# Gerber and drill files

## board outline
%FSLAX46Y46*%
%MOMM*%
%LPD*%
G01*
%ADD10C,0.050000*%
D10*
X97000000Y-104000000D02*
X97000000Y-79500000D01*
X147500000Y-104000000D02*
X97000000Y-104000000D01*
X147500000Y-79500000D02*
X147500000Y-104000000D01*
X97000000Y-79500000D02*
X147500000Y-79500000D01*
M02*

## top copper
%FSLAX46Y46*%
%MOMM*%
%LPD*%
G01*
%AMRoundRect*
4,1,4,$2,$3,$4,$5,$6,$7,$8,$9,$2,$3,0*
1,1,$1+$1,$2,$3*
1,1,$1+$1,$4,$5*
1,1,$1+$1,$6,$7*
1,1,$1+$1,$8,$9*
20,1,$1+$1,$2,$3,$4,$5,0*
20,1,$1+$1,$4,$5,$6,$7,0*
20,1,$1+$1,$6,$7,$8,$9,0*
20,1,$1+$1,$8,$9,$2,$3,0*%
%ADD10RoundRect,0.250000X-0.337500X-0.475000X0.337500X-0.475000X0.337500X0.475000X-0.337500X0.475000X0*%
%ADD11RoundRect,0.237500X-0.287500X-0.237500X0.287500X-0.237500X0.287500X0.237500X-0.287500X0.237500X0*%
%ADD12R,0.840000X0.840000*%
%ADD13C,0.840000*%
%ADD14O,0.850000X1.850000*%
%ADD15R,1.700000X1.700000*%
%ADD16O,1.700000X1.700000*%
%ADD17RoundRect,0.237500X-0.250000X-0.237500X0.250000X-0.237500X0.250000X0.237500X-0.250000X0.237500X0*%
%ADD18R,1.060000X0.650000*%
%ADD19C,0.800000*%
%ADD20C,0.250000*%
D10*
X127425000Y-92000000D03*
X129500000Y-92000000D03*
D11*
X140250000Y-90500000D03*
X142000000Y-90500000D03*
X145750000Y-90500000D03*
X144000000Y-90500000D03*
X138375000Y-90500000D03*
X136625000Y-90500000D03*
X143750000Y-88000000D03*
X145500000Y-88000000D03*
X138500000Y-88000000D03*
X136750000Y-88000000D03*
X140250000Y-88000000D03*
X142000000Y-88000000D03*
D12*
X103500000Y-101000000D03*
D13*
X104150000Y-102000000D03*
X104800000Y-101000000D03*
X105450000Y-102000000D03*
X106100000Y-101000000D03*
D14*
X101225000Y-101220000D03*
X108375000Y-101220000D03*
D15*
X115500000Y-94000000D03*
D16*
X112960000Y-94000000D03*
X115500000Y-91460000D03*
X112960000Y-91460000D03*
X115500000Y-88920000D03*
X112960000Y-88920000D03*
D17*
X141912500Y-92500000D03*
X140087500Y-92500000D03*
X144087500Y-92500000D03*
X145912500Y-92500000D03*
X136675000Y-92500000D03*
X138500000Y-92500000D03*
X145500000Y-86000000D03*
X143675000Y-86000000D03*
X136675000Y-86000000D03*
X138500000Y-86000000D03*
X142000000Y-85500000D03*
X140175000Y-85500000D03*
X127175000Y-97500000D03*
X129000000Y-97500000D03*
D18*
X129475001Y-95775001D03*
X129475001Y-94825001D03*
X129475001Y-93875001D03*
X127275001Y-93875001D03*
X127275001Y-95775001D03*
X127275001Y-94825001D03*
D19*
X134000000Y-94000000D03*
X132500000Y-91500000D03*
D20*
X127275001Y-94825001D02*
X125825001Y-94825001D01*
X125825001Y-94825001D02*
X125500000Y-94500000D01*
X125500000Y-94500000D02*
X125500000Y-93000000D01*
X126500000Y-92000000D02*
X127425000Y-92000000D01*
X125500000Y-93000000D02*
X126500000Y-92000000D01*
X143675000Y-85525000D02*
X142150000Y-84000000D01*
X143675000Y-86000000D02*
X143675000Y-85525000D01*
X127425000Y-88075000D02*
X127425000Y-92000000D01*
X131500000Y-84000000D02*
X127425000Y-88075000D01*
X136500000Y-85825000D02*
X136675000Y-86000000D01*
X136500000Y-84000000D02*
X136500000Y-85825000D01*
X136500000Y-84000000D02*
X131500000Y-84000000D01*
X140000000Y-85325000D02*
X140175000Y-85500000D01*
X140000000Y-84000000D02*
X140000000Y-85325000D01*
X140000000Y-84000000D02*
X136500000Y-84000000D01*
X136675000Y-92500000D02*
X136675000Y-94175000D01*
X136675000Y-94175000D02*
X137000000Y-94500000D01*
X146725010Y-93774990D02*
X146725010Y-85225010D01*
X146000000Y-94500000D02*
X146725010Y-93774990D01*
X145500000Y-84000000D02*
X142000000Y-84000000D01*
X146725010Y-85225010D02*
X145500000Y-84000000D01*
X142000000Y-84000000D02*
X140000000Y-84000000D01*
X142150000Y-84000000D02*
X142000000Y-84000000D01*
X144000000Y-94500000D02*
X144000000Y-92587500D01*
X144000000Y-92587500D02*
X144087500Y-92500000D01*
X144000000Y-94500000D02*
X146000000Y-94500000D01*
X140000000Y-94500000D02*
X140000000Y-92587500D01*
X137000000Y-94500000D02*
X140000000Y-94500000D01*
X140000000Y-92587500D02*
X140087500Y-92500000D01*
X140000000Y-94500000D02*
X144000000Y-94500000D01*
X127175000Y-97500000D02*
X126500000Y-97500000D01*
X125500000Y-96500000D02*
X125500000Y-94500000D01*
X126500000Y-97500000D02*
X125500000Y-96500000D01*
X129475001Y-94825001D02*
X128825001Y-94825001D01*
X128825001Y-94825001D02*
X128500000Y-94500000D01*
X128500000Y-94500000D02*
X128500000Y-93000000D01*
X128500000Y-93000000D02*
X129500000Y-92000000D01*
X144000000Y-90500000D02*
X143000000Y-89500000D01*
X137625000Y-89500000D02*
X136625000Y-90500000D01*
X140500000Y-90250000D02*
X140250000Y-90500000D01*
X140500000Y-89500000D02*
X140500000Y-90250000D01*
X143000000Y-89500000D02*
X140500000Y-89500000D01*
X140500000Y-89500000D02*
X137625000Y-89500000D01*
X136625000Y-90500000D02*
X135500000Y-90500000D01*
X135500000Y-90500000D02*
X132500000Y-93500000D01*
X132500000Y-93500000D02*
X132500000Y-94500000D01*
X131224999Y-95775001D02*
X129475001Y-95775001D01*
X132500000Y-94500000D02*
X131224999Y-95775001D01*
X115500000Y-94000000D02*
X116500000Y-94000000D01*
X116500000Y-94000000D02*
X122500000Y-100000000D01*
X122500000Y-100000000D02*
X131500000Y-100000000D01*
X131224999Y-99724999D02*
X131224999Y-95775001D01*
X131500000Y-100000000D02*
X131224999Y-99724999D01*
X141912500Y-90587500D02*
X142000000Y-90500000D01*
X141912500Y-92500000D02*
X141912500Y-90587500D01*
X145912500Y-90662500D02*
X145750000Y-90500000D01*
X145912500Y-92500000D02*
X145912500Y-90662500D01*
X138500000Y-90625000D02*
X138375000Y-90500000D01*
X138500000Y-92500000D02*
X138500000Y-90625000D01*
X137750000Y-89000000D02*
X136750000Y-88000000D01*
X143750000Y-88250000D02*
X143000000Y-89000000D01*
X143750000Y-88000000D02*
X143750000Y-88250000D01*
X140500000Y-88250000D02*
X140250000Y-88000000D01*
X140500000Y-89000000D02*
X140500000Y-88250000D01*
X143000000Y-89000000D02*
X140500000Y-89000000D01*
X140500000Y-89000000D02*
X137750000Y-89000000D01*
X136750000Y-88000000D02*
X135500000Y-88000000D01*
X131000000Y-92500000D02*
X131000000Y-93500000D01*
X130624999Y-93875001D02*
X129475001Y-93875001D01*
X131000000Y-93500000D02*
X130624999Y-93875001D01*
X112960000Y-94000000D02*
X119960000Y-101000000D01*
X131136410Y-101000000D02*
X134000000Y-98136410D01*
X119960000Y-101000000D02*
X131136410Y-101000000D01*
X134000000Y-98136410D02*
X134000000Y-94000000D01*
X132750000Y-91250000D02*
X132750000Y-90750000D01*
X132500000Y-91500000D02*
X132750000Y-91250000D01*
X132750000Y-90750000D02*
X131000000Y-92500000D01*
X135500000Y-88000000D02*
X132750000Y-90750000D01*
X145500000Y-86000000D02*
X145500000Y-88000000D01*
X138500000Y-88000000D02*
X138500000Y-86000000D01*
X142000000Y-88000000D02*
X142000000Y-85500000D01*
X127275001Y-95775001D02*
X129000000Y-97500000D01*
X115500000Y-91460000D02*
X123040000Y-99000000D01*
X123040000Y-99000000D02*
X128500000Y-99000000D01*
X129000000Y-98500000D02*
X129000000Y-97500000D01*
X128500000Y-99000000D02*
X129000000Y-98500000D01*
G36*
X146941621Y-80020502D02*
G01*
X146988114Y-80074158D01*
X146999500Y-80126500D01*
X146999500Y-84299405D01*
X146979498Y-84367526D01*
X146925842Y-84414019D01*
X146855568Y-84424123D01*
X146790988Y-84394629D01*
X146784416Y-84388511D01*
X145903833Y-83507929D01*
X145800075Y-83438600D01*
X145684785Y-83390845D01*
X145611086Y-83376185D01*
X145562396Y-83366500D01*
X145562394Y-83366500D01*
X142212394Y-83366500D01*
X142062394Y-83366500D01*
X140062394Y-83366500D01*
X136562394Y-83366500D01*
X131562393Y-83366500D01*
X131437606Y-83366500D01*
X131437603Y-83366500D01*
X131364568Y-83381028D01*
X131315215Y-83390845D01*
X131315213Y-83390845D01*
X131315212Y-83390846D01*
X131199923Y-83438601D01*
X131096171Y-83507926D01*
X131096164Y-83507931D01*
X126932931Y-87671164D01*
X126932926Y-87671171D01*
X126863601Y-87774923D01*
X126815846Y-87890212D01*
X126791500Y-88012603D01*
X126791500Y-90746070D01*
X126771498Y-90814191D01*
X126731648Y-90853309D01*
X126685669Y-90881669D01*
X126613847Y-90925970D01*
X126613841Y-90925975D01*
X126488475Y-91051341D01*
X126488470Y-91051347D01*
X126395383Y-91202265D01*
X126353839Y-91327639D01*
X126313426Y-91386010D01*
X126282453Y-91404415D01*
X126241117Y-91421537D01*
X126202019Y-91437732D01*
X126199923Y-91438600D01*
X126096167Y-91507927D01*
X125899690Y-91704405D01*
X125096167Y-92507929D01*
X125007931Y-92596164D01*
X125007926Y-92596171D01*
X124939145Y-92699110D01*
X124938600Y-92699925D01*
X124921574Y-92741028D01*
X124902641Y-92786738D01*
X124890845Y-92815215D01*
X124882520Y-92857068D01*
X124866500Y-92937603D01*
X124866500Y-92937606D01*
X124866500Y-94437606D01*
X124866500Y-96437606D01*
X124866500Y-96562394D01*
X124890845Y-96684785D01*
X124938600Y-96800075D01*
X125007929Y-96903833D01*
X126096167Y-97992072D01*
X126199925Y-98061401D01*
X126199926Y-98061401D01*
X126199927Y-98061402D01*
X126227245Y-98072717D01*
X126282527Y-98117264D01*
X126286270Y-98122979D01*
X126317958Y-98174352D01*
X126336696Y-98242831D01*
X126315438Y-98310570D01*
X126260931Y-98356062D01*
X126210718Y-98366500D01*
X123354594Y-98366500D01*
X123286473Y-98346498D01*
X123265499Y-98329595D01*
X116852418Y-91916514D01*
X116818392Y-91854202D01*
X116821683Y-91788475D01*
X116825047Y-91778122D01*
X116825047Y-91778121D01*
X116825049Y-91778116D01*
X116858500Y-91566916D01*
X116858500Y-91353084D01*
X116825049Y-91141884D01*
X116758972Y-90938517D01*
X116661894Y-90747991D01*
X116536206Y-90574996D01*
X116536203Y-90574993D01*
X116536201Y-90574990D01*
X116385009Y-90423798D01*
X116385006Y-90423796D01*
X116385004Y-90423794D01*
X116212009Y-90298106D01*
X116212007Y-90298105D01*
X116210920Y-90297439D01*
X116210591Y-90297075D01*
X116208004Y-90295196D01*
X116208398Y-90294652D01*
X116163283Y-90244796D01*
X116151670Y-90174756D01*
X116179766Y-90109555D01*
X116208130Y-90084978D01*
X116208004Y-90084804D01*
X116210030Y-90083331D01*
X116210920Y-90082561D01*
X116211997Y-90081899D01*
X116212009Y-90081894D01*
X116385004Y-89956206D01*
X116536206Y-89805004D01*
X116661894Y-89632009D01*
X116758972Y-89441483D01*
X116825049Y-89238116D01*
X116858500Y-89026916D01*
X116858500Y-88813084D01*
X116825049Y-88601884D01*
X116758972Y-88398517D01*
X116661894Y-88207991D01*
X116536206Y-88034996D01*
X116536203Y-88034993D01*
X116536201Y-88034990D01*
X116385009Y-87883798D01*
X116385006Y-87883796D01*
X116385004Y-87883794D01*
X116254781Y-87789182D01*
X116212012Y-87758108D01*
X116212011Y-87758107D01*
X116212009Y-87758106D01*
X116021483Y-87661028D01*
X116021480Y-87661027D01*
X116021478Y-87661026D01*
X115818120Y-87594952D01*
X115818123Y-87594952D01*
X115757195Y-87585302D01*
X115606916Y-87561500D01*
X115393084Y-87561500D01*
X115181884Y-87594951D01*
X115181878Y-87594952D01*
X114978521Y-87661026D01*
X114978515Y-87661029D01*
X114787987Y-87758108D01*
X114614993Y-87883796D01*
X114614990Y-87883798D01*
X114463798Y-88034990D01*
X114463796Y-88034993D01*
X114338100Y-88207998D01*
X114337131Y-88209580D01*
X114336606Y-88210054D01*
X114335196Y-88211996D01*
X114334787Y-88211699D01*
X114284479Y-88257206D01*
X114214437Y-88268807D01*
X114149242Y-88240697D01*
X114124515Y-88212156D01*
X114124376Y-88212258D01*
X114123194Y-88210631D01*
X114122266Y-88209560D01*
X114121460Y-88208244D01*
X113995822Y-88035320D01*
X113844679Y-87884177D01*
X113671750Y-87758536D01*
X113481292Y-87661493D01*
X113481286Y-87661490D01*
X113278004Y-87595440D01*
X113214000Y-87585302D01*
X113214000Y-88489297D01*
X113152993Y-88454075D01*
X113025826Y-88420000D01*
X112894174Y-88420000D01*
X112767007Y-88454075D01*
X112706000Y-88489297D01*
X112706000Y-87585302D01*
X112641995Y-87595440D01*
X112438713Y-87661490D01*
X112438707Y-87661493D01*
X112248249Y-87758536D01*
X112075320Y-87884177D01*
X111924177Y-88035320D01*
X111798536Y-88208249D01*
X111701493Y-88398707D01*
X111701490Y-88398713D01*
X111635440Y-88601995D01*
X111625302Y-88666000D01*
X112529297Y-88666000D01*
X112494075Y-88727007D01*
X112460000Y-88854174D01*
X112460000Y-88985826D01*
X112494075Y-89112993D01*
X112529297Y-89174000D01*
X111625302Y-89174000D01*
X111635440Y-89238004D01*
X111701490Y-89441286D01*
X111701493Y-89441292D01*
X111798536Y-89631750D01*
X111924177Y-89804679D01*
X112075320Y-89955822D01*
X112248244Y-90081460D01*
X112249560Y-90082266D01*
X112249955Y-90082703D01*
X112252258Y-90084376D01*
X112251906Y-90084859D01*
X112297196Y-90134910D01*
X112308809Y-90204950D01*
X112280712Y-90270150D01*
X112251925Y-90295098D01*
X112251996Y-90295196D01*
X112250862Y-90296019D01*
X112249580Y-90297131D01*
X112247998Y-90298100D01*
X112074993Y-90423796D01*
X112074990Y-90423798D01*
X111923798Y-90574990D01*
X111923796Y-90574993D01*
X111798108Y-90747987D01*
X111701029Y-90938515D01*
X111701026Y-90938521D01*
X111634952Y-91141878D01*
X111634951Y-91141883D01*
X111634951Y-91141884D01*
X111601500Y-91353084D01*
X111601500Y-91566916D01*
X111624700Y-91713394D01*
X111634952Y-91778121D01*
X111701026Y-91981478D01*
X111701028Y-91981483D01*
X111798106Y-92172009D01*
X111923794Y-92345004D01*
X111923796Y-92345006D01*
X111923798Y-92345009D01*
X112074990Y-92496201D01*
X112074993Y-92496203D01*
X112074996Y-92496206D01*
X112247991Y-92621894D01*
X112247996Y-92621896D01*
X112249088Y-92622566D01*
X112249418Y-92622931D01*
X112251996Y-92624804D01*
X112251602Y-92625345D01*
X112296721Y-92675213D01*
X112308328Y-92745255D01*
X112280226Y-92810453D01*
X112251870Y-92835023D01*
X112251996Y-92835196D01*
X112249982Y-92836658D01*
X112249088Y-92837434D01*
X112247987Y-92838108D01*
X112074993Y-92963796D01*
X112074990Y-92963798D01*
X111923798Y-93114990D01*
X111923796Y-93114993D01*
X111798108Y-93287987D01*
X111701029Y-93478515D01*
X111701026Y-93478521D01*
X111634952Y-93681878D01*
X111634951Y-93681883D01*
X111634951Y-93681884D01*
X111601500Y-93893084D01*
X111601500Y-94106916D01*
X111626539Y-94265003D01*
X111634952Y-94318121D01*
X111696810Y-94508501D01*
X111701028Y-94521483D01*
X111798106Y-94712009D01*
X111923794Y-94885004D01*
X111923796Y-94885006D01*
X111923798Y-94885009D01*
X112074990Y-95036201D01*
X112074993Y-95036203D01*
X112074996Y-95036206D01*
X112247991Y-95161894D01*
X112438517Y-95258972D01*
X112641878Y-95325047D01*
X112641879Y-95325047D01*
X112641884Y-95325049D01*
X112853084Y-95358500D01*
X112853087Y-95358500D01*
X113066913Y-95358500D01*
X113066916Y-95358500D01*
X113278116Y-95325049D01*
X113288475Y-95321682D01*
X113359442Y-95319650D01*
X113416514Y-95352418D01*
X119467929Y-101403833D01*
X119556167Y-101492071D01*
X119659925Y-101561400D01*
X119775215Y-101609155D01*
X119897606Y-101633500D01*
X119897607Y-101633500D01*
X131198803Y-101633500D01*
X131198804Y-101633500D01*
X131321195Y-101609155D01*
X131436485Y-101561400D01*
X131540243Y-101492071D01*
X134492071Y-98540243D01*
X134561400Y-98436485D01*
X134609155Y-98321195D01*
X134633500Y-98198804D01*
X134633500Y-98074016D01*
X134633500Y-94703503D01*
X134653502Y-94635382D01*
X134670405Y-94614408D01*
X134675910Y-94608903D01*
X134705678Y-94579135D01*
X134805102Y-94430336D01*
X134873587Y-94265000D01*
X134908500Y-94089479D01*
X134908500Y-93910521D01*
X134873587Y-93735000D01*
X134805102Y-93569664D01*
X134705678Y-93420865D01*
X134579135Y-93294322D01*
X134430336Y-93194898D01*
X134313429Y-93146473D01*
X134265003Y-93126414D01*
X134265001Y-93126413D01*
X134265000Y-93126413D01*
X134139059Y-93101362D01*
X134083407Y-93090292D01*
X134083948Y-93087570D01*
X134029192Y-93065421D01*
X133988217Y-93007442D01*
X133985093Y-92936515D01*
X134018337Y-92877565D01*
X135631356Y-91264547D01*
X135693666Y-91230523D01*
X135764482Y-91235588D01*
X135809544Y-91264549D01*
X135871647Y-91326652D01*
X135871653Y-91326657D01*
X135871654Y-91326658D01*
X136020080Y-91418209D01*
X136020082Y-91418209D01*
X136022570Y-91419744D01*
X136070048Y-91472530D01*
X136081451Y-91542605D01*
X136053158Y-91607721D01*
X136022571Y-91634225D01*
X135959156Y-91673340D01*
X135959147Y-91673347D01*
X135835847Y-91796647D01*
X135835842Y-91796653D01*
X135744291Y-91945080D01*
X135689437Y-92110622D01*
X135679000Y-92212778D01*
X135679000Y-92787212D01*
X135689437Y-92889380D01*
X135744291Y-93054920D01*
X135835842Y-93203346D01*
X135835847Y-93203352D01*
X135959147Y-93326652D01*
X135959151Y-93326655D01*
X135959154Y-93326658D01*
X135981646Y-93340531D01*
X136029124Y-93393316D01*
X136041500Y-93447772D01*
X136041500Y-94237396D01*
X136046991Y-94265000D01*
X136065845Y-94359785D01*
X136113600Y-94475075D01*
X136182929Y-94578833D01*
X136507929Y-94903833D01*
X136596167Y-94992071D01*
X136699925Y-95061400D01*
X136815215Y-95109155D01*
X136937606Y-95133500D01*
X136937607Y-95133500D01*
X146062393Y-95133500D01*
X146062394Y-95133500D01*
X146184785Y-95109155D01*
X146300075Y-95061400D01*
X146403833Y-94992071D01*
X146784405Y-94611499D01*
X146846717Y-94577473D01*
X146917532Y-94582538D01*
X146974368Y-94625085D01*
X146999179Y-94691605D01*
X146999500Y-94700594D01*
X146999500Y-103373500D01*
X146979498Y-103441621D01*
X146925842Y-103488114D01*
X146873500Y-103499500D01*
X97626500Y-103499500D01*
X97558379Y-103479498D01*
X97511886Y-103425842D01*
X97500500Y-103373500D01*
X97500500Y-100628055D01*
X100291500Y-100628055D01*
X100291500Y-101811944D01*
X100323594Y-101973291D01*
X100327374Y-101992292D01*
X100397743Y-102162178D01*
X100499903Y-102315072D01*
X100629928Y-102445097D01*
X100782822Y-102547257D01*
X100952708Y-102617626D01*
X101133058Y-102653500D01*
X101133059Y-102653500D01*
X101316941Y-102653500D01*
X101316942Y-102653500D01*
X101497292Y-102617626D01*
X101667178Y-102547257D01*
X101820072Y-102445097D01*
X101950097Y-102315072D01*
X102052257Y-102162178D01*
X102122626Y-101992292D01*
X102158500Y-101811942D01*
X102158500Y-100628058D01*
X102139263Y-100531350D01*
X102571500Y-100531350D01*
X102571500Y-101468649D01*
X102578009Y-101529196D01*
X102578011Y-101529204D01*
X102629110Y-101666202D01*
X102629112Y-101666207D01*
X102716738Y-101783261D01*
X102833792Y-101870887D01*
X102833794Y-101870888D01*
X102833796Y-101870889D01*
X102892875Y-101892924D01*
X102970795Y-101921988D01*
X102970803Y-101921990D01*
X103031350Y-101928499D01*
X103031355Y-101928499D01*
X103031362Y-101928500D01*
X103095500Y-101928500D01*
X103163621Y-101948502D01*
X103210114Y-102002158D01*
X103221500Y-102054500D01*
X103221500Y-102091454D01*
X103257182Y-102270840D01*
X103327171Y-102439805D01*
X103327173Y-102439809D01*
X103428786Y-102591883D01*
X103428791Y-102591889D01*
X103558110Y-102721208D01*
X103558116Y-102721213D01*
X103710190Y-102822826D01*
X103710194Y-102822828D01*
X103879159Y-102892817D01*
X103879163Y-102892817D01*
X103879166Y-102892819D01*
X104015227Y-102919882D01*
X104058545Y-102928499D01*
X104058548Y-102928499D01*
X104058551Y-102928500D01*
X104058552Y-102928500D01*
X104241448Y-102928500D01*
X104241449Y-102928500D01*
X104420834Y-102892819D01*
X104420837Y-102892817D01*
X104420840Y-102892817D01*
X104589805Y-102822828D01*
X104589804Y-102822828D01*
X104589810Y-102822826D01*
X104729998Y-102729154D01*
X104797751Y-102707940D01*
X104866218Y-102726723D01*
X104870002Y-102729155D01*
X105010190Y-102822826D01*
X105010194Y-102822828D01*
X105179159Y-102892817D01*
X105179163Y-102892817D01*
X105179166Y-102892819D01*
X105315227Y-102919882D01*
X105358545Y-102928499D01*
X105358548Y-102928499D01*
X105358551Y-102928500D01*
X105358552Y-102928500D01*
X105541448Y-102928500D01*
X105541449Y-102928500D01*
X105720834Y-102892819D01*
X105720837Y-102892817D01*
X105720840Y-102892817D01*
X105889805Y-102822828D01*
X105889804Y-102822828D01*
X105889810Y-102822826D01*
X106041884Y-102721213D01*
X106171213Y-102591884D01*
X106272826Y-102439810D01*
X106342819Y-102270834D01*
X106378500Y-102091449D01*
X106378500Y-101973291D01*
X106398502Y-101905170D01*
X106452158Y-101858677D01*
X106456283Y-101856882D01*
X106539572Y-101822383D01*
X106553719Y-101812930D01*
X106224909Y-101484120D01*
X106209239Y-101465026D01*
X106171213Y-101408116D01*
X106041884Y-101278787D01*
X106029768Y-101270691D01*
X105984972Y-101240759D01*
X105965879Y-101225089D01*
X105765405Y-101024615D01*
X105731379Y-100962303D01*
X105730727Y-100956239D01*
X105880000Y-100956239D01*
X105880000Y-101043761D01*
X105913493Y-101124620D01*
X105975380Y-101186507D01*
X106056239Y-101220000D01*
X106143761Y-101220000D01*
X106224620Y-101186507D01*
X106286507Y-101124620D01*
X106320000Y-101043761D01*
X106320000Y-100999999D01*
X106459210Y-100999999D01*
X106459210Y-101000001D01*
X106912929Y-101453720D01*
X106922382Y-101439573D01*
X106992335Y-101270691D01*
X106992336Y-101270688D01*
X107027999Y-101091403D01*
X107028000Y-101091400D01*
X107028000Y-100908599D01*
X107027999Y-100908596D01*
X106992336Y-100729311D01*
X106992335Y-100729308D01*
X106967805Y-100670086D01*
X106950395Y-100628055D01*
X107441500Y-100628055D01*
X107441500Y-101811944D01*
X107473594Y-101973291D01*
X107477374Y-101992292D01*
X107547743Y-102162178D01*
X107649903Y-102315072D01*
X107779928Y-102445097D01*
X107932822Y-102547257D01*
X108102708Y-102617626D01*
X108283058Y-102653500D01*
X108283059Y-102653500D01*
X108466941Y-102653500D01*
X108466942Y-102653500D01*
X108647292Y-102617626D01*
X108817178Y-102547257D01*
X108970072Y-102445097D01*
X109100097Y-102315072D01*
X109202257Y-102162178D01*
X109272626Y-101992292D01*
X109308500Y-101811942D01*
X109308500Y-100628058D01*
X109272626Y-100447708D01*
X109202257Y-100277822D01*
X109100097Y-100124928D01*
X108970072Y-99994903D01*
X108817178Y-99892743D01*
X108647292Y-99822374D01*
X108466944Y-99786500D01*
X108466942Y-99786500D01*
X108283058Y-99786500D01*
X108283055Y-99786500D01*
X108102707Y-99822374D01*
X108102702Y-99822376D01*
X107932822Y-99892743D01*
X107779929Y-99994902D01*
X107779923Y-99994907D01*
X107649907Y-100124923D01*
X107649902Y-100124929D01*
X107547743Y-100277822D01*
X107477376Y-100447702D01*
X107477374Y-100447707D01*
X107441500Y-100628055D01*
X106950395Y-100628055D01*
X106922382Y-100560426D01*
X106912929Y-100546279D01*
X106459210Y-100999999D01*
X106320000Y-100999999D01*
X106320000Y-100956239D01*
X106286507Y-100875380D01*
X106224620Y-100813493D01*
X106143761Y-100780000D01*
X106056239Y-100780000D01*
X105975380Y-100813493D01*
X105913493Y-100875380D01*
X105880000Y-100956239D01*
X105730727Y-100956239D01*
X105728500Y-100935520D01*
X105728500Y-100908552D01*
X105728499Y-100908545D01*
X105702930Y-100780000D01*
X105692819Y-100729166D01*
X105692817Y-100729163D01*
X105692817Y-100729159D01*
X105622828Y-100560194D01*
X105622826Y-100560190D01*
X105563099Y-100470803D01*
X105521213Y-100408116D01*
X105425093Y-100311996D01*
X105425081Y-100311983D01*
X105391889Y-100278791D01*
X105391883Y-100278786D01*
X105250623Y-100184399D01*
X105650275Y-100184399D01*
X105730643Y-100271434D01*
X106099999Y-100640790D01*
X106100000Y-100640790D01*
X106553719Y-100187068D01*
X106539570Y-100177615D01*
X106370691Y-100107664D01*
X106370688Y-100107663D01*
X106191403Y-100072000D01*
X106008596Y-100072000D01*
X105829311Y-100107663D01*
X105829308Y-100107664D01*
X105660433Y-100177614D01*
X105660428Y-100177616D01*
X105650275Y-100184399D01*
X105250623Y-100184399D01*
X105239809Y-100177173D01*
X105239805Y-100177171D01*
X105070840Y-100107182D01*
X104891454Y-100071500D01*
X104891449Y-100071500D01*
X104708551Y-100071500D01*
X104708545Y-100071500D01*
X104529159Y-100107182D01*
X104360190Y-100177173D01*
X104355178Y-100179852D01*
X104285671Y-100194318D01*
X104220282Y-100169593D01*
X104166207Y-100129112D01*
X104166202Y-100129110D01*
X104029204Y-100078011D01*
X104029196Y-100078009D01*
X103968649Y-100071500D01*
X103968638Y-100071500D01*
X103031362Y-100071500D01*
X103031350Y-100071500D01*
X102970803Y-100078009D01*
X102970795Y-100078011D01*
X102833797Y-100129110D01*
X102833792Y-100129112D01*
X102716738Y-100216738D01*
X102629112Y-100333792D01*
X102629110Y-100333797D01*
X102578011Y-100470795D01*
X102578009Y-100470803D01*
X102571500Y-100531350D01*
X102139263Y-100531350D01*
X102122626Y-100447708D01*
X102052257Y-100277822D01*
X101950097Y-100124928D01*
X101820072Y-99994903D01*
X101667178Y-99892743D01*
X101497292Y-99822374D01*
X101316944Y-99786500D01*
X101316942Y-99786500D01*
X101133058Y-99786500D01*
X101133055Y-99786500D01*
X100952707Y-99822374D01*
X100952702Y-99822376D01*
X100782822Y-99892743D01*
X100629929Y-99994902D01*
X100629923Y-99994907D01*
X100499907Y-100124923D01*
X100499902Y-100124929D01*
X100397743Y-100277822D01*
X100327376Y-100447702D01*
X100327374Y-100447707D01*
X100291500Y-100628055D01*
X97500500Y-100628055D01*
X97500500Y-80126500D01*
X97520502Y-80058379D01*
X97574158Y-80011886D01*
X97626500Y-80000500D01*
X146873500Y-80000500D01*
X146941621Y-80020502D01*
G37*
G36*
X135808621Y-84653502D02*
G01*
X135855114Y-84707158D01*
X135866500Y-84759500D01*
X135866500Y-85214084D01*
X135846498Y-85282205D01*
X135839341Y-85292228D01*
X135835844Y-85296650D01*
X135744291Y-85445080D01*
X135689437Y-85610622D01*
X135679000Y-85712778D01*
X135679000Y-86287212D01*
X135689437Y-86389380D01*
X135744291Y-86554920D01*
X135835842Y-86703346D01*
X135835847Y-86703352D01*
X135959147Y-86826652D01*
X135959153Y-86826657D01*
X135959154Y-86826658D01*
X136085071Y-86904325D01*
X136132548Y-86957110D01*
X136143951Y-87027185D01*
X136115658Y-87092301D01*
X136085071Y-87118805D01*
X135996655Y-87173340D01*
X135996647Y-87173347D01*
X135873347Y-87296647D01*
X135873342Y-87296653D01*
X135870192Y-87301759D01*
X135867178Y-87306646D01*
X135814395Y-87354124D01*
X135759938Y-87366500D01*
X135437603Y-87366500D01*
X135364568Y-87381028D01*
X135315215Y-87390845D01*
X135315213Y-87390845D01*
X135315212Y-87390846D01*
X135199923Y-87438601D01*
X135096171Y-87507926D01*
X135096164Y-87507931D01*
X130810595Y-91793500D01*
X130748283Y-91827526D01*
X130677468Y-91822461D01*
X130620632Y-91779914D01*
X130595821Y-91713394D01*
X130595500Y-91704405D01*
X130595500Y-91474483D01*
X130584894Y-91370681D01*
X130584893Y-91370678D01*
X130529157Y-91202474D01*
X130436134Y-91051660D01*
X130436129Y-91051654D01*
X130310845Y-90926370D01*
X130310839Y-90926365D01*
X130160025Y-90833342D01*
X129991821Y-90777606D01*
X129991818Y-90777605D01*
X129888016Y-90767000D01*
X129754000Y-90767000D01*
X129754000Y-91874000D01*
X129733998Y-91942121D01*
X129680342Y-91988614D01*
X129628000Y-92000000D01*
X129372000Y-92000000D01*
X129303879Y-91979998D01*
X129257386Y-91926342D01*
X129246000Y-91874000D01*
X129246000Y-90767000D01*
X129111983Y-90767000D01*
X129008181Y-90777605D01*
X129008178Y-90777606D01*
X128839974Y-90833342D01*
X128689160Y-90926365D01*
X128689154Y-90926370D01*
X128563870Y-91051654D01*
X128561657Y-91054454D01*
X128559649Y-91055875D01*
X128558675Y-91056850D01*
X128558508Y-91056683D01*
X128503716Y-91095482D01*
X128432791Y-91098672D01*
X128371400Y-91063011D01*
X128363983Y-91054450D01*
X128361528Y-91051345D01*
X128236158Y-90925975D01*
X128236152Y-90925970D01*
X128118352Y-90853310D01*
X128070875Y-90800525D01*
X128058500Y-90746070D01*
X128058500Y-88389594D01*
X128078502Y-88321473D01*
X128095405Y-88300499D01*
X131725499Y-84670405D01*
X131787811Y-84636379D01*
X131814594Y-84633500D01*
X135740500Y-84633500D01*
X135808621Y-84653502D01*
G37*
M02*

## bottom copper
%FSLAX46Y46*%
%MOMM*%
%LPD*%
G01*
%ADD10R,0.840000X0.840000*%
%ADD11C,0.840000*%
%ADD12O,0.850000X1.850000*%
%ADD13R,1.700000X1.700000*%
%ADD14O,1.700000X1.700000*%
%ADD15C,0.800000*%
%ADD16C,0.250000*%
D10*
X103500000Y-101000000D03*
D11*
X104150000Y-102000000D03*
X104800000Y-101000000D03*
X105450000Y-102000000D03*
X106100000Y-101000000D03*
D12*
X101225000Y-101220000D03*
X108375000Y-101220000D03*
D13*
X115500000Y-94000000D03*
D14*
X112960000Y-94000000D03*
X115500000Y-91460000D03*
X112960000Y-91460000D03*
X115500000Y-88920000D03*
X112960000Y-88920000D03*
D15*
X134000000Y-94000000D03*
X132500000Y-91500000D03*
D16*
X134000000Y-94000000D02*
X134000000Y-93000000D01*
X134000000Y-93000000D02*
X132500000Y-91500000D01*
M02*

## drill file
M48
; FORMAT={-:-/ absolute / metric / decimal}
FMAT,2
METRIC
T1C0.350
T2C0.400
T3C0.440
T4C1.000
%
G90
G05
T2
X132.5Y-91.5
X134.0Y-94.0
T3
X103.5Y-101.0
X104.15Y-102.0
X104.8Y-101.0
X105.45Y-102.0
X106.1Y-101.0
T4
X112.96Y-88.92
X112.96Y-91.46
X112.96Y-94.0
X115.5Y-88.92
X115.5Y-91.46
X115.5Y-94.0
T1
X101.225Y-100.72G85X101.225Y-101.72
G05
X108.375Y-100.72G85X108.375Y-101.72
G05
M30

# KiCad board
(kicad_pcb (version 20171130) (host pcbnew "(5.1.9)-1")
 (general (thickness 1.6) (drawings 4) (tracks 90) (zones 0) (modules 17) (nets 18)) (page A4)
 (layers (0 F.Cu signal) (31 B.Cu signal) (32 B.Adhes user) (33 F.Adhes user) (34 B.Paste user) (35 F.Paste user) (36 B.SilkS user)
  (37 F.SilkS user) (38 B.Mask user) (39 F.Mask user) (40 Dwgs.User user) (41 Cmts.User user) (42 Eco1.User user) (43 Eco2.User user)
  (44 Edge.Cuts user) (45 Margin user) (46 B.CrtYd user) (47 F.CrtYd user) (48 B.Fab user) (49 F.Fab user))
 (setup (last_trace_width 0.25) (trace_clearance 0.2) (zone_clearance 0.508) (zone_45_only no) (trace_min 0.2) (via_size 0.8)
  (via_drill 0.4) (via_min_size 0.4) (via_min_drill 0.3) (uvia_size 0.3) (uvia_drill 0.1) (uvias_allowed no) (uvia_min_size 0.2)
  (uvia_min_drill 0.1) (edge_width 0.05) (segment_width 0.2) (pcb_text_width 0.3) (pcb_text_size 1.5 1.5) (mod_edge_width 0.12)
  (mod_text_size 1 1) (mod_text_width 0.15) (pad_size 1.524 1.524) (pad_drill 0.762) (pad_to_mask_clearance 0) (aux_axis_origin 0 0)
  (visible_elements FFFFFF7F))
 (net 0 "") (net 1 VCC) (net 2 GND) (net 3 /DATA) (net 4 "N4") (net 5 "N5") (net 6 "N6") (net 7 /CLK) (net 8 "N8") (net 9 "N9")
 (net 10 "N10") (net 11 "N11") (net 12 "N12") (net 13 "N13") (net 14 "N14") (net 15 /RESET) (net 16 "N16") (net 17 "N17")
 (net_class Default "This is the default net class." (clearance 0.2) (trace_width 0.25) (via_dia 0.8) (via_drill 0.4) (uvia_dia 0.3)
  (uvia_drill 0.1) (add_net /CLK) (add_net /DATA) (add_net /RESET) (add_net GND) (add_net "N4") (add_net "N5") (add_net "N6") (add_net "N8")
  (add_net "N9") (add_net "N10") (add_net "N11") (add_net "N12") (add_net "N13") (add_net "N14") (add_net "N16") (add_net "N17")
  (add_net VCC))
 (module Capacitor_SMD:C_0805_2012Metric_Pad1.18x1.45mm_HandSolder (layer F.Cu) (at 128.4625 92)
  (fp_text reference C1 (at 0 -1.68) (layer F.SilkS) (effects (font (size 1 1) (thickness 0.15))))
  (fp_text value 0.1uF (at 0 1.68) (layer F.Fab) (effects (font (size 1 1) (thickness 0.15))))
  (pad 1 smd roundrect (at -1.0375 0) (size 1.175 1.45) (layers F.Cu F.Paste F.Mask) (roundrect_rratio 0.212766) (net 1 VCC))
  (pad 2 smd roundrect (at 1.0375 0) (size 1.175 1.45) (layers F.Cu F.Paste F.Mask) (roundrect_rratio 0.212766) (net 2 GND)))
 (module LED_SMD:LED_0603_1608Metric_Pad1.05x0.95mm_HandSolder (layer F.Cu) (at 141.125 90.5)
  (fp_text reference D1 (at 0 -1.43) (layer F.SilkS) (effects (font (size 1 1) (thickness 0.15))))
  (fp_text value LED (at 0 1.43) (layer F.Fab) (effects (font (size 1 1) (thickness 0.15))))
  (pad 1 smd roundrect (at -0.875 0) (size 1.05 0.95) (layers F.Cu F.Paste F.Mask) (roundrect_rratio 0.25) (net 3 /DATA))
  (pad 2 smd roundrect (at 0.875 0) (size 1.05 0.95) (layers F.Cu F.Paste F.Mask) (roundrect_rratio 0.25) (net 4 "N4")))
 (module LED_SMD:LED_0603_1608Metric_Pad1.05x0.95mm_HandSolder (layer F.Cu) (at 144.875 90.5)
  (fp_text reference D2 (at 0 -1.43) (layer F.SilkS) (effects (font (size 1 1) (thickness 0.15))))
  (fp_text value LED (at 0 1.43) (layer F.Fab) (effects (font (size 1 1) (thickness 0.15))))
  (pad 2 smd roundrect (at 0.875 0) (size 1.05 0.95) (layers F.Cu F.Paste F.Mask) (roundrect_rratio 0.25) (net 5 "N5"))
  (pad 1 smd roundrect (at -0.875 0) (size 1.05 0.95) (layers F.Cu F.Paste F.Mask) (roundrect_rratio 0.25) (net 3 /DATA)))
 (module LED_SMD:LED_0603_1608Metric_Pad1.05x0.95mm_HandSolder (layer F.Cu) (at 137.5 90.5)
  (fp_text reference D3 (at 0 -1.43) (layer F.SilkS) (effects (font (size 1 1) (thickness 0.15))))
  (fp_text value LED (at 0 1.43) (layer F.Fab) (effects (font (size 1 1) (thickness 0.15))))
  (pad 2 smd roundrect (at 0.875 0) (size 1.05 0.95) (layers F.Cu F.Paste F.Mask) (roundrect_rratio 0.25) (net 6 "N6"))
  (pad 1 smd roundrect (at -0.875 0) (size 1.05 0.95) (layers F.Cu F.Paste F.Mask) (roundrect_rratio 0.25) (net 3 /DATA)))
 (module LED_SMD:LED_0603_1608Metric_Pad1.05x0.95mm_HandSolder (layer F.Cu) (at 144.625 88)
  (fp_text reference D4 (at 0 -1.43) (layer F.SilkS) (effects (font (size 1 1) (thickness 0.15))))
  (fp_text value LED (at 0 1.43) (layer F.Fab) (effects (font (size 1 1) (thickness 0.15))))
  (pad 1 smd roundrect (at -0.875 0) (size 1.05 0.95) (layers F.Cu F.Paste F.Mask) (roundrect_rratio 0.25) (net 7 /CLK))
  (pad 2 smd roundrect (at 0.875 0) (size 1.05 0.95) (layers F.Cu F.Paste F.Mask) (roundrect_rratio 0.25) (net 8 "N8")))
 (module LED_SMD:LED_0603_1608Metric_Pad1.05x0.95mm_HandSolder (layer F.Cu) (at 137.625 88)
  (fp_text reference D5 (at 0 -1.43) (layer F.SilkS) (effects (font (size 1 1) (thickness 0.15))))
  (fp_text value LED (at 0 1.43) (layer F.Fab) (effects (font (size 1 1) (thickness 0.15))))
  (pad 2 smd roundrect (at 0.875 0) (size 1.05 0.95) (layers F.Cu F.Paste F.Mask) (roundrect_rratio 0.25) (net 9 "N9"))
  (pad 1 smd roundrect (at -0.875 0) (size 1.05 0.95) (layers F.Cu F.Paste F.Mask) (roundrect_rratio 0.25) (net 7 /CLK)))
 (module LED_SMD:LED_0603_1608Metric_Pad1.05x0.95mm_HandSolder (layer F.Cu) (at 141.125 88)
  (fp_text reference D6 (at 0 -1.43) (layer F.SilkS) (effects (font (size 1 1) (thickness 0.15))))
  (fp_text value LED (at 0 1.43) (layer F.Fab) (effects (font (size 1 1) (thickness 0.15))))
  (pad 1 smd roundrect (at -0.875 0) (size 1.05 0.95) (layers F.Cu F.Paste F.Mask) (roundrect_rratio 0.25) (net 7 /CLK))
  (pad 2 smd roundrect (at 0.875 0) (size 1.05 0.95) (layers F.Cu F.Paste F.Mask) (roundrect_rratio 0.25) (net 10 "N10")))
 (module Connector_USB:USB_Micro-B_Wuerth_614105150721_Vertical (layer F.Cu) (at 103.5 101)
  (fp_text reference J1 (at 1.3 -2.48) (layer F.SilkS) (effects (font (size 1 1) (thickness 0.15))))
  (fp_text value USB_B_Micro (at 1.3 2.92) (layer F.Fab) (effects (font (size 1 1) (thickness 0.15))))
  (pad 1 thru_hole rect (at 0 0) (size 0.84 0.84) (drill 0.44) (layers *.Cu *.Mask) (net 1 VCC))
  (pad 2 thru_hole circle (at 0.65 1) (size 0.84 0.84) (drill 0.44) (layers *.Cu *.Mask) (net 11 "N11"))
  (pad 3 thru_hole circle (at 1.3 0) (size 0.84 0.84) (drill 0.44) (layers *.Cu *.Mask) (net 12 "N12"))
  (pad 4 thru_hole circle (at 1.95 1) (size 0.84 0.84) (drill 0.44) (layers *.Cu *.Mask) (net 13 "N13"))
  (pad 5 thru_hole circle (at 2.6 0) (size 0.84 0.84) (drill 0.44) (layers *.Cu *.Mask) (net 2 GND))
  (pad 6 thru_hole oval (at -2.275 0.22) (size 0.85 1.85) (drill oval 0.35 1.35) (layers *.Cu *.Mask) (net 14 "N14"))
  (pad 6 thru_hole oval (at 4.875 0.22) (size 0.85 1.85) (drill oval 0.35 1.35) (layers *.Cu *.Mask) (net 14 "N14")))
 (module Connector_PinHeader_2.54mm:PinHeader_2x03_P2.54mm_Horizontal (layer F.Cu) (at 115.5 94 180)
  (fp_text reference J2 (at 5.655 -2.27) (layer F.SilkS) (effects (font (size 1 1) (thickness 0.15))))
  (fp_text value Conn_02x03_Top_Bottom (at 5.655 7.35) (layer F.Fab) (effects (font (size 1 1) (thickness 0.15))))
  (pad 1 thru_hole rect (at 0 0 180) (size 1.7 1.7) (drill 1) (layers *.Cu *.Mask) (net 3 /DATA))
  (pad 2 thru_hole oval (at 2.54 0 180) (size 1.7 1.7) (drill 1) (layers *.Cu *.Mask) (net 7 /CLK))
  (pad 3 thru_hole oval (at 0 2.54 180) (size 1.7 1.7) (drill 1) (layers *.Cu *.Mask) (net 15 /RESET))
  (pad 4 thru_hole oval (at 2.54 2.54 180) (size 1.7 1.7) (drill 1) (layers *.Cu *.Mask) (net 1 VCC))
  (pad 5 thru_hole oval (at 0 5.08 180) (size 1.7 1.7) (drill 1) (layers *.Cu *.Mask) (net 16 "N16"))
  (pad 6 thru_hole oval (at 2.54 5.08 180) (size 1.7 1.7) (drill 1) (layers *.Cu *.Mask) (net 2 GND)))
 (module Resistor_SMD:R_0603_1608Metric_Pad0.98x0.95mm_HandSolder (layer F.Cu) (at 141 92.5)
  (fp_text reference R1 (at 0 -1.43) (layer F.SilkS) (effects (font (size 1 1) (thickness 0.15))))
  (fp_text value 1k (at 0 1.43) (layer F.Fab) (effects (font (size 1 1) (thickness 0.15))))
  (pad 2 smd roundrect (at 0.9125 0) (size 0.975 0.95) (layers F.Cu F.Paste F.Mask) (roundrect_rratio 0.25) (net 4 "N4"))
  (pad 1 smd roundrect (at -0.9125 0) (size 0.975 0.95) (layers F.Cu F.Paste F.Mask) (roundrect_rratio 0.25) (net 1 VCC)))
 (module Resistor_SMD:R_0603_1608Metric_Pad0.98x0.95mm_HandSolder (layer F.Cu) (at 145 92.5)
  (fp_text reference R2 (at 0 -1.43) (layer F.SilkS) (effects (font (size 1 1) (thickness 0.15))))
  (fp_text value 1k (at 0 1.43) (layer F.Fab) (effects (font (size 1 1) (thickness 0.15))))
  (pad 1 smd roundrect (at -0.9125 0) (size 0.975 0.95) (layers F.Cu F.Paste F.Mask) (roundrect_rratio 0.25) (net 1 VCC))
  (pad 2 smd roundrect (at 0.9125 0) (size 0.975 0.95) (layers F.Cu F.Paste F.Mask) (roundrect_rratio 0.25) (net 5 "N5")))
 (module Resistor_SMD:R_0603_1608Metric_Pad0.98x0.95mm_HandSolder (layer F.Cu) (at 137.5875 92.5)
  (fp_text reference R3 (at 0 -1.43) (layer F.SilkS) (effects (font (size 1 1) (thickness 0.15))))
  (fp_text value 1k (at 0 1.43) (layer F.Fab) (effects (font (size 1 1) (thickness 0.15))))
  (pad 1 smd roundrect (at -0.9125 0) (size 0.975 0.95) (layers F.Cu F.Paste F.Mask) (roundrect_rratio 0.25) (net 1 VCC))
  (pad 2 smd roundrect (at 0.9125 0) (size 0.975 0.95) (layers F.Cu F.Paste F.Mask) (roundrect_rratio 0.25) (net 6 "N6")))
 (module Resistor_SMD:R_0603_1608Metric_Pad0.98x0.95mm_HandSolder (layer F.Cu) (at 144.5875 86)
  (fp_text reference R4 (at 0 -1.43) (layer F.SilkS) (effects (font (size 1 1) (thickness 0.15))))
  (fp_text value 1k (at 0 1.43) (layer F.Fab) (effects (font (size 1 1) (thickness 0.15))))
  (pad 2 smd roundrect (at 0.9125 0) (size 0.975 0.95) (layers F.Cu F.Paste F.Mask) (roundrect_rratio 0.25) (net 8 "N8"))
  (pad 1 smd roundrect (at -0.9125 0) (size 0.975 0.95) (layers F.Cu F.Paste F.Mask) (roundrect_rratio 0.25) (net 1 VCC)))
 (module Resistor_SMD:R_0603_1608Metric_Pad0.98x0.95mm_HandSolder (layer F.Cu) (at 137.5875 86)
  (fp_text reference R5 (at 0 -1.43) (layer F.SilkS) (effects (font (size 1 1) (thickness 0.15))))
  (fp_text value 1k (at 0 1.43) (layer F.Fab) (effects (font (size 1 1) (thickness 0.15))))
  (pad 1 smd roundrect (at -0.9125 0) (size 0.975 0.95) (layers F.Cu F.Paste F.Mask) (roundrect_rratio 0.25) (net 1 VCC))
  (pad 2 smd roundrect (at 0.9125 0) (size 0.975 0.95) (layers F.Cu F.Paste F.Mask) (roundrect_rratio 0.25) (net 9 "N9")))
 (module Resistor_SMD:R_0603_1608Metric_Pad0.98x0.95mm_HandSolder (layer F.Cu) (at 141.0875 85.5)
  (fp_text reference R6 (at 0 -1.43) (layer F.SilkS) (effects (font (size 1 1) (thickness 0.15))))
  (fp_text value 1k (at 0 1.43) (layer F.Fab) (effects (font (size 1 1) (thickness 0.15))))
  (pad 2 smd roundrect (at 0.9125 0) (size 0.975 0.95) (layers F.Cu F.Paste F.Mask) (roundrect_rratio 0.25) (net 10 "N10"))
  (pad 1 smd roundrect (at -0.9125 0) (size 0.975 0.95) (layers F.Cu F.Paste F.Mask) (roundrect_rratio 0.25) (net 1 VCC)))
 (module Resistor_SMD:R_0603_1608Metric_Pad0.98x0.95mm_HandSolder (layer F.Cu) (at 128.0875 97.5)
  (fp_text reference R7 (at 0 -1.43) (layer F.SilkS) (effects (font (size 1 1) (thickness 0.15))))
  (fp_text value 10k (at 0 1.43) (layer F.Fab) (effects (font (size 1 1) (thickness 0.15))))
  (pad 1 smd roundrect (at -0.9125 0) (size 0.975 0.95) (layers F.Cu F.Paste F.Mask) (roundrect_rratio 0.25) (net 1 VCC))
  (pad 2 smd roundrect (at 0.9125 0) (size 0.975 0.95) (layers F.Cu F.Paste F.Mask) (roundrect_rratio 0.25) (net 15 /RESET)))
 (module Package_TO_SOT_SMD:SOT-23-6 (layer F.Cu) (at 128.375001 94.825001 180)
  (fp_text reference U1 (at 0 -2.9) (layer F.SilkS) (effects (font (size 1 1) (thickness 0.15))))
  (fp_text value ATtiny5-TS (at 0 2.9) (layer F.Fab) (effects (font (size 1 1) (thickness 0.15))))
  (pad 1 smd rect (at -1.1 -0.95 180) (size 1.06 0.65) (layers F.Cu F.Paste F.Mask) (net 3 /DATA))
  (pad 2 smd rect (at -1.1 0 180) (size 1.06 0.65) (layers F.Cu F.Paste F.Mask) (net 2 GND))
  (pad 3 smd rect (at -1.1 0.95 180) (size 1.06 0.65) (layers F.Cu F.Paste F.Mask) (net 7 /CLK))
  (pad 4 smd rect (at 1.1 0.95 180) (size 1.06 0.65) (layers F.Cu F.Paste F.Mask) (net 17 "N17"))
  (pad 6 smd rect (at 1.1 -0.95 180) (size 1.06 0.65) (layers F.Cu F.Paste F.Mask) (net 15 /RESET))
  (pad 5 smd rect (at 1.1 0 180) (size 1.06 0.65) (layers F.Cu F.Paste F.Mask) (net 1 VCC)))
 (gr_line (start 97 104) (end 97 79.5) (layer Edge.Cuts) (width 0.05))
 (gr_line (start 147.5 104) (end 97 104) (layer Edge.Cuts) (width 0.05))
 (gr_line (start 147.5 79.5) (end 147.5 104) (layer Edge.Cuts) (width 0.05))
 (gr_line (start 97 79.5) (end 147.5 79.5) (layer Edge.Cuts) (width 0.05))
 (segment (start 127.275001 94.825001) (end 125.825001 94.825001) (width 0.25) (layer F.Cu) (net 1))
 (segment (start 125.825001 94.825001) (end 125.5 94.5) (width 0.25) (layer F.Cu) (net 1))
 (segment (start 125.5 94.5) (end 125.5 93) (width 0.25) (layer F.Cu) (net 1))
 (segment (start 126.5 92) (end 127.425 92) (width 0.25) (layer F.Cu) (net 1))
 (segment (start 125.5 93) (end 126.5 92) (width 0.25) (layer F.Cu) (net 1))
 (segment (start 143.675 85.525) (end 142.15 84) (width 0.25) (layer F.Cu) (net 1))
 (segment (start 143.675 86) (end 143.675 85.525) (width 0.25) (layer F.Cu) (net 1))
 (segment (start 127.425 88.075) (end 127.425 92) (width 0.25) (layer F.Cu) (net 1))
 (segment (start 131.5 84) (end 127.425 88.075) (width 0.25) (layer F.Cu) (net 1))
 (segment (start 136.5 85.825) (end 136.675 86) (width 0.25) (layer F.Cu) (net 1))
 (segment (start 136.5 84) (end 136.5 85.825) (width 0.25) (layer F.Cu) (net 1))
 (segment (start 136.5 84) (end 131.5 84) (width 0.25) (layer F.Cu) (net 1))
 (segment (start 140 85.325) (end 140.175 85.5) (width 0.25) (layer F.Cu) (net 1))
 (segment (start 140 84) (end 140 85.325) (width 0.25) (layer F.Cu) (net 1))
 (segment (start 140 84) (end 136.5 84) (width 0.25) (layer F.Cu) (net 1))
 (segment (start 136.675 92.5) (end 136.675 94.175) (width 0.25) (layer F.Cu) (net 1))
 (segment (start 136.675 94.175) (end 137 94.5) (width 0.25) (layer F.Cu) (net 1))
 (segment (start 146.72501 93.77499) (end 146.72501 85.22501) (width 0.25) (layer F.Cu) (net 1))
 (segment (start 146 94.5) (end 146.72501 93.77499) (width 0.25) (layer F.Cu) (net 1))
 (segment (start 145.5 84) (end 142 84) (width 0.25) (layer F.Cu) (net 1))
 (segment (start 146.72501 85.22501) (end 145.5 84) (width 0.25) (layer F.Cu) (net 1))
 (segment (start 142 84) (end 140 84) (width 0.25) (layer F.Cu) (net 1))
 (segment (start 142.15 84) (end 142 84) (width 0.25) (layer F.Cu) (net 1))
 (segment (start 144 94.5) (end 144 92.5875) (width 0.25) (layer F.Cu) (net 1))
 (segment (start 144 92.5875) (end 144.0875 92.5) (width 0.25) (layer F.Cu) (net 1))
 (segment (start 144 94.5) (end 146 94.5) (width 0.25) (layer F.Cu) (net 1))
 (segment (start 140 94.5) (end 140 92.5875) (width 0.25) (layer F.Cu) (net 1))
 (segment (start 137 94.5) (end 140 94.5) (width 0.25) (layer F.Cu) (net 1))
 (segment (start 140 92.5875) (end 140.0875 92.5) (width 0.25) (layer F.Cu) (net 1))
 (segment (start 140 94.5) (end 144 94.5) (width 0.25) (layer F.Cu) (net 1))
 (segment (start 127.175 97.5) (end 126.5 97.5) (width 0.25) (layer F.Cu) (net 1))
 (segment (start 125.5 96.5) (end 125.5 94.5) (width 0.25) (layer F.Cu) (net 1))
 (segment (start 126.5 97.5) (end 125.5 96.5) (width 0.25) (layer F.Cu) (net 1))
 (segment (start 129.475001 94.825001) (end 128.825001 94.825001) (width 0.25) (layer F.Cu) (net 2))
 (segment (start 128.825001 94.825001) (end 128.5 94.5) (width 0.25) (layer F.Cu) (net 2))
 (segment (start 128.5 94.5) (end 128.5 93) (width 0.25) (layer F.Cu) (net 2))
 (segment (start 128.5 93) (end 129.5 92) (width 0.25) (layer F.Cu) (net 2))
 (segment (start 144 90.5) (end 143 89.5) (width 0.25) (layer F.Cu) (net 3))
 (segment (start 137.625 89.5) (end 136.625 90.5) (width 0.25) (layer F.Cu) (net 3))
 (segment (start 140.5 90.25) (end 140.25 90.5) (width 0.25) (layer F.Cu) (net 3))
 (segment (start 140.5 89.5) (end 140.5 90.25) (width 0.25) (layer F.Cu) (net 3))
 (segment (start 143 89.5) (end 140.5 89.5) (width 0.25) (layer F.Cu) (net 3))
 (segment (start 140.5 89.5) (end 137.625 89.5) (width 0.25) (layer F.Cu) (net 3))
 (segment (start 136.625 90.5) (end 135.5 90.5) (width 0.25) (layer F.Cu) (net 3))
 (segment (start 135.5 90.5) (end 132.5 93.5) (width 0.25) (layer F.Cu) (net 3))
 (segment (start 132.5 93.5) (end 132.5 94.5) (width 0.25) (layer F.Cu) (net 3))
 (segment (start 131.224999 95.775001) (end 129.475001 95.775001) (width 0.25) (layer F.Cu) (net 3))
 (segment (start 132.5 94.5) (end 131.224999 95.775001) (width 0.25) (layer F.Cu) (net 3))
 (segment (start 115.5 94) (end 116.5 94) (width 0.25) (layer F.Cu) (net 3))
 (segment (start 116.5 94) (end 122.5 100) (width 0.25) (layer F.Cu) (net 3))
 (segment (start 122.5 100) (end 131.5 100) (width 0.25) (layer F.Cu) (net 3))
 (segment (start 131.224999 99.724999) (end 131.224999 95.775001) (width 0.25) (layer F.Cu) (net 3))
 (segment (start 131.5 100) (end 131.224999 99.724999) (width 0.25) (layer F.Cu) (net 3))
 (segment (start 141.9125 90.5875) (end 142 90.5) (width 0.25) (layer F.Cu) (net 4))
 (segment (start 141.9125 92.5) (end 141.9125 90.5875) (width 0.25) (layer F.Cu) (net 4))
 (segment (start 145.9125 90.6625) (end 145.75 90.5) (width 0.25) (layer F.Cu) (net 5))
 (segment (start 145.9125 92.5) (end 145.9125 90.6625) (width 0.25) (layer F.Cu) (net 5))
 (segment (start 138.5 90.625) (end 138.375 90.5) (width 0.25) (layer F.Cu) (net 6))
 (segment (start 138.5 92.5) (end 138.5 90.625) (width 0.25) (layer F.Cu) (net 6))
 (segment (start 137.75 89) (end 136.75 88) (width 0.25) (layer F.Cu) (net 7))
 (segment (start 143.75 88.25) (end 143 89) (width 0.25) (layer F.Cu) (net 7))
 (segment (start 143.75 88) (end 143.75 88.25) (width 0.25) (layer F.Cu) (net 7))
 (segment (start 140.5 88.25) (end 140.25 88) (width 0.25) (layer F.Cu) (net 7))
 (segment (start 140.5 89) (end 140.5 88.25) (width 0.25) (layer F.Cu) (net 7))
 (segment (start 143 89) (end 140.5 89) (width 0.25) (layer F.Cu) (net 7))
 (segment (start 140.5 89) (end 137.75 89) (width 0.25) (layer F.Cu) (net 7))
 (segment (start 136.75 88) (end 135.5 88) (width 0.25) (layer F.Cu) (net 7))
 (segment (start 131 92.5) (end 131 93.5) (width 0.25) (layer F.Cu) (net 7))
 (segment (start 130.624999 93.875001) (end 129.475001 93.875001) (width 0.25) (layer F.Cu) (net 7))
 (segment (start 131 93.5) (end 130.624999 93.875001) (width 0.25) (layer F.Cu) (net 7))
 (segment (start 112.96 94) (end 119.96 101) (width 0.25) (layer F.Cu) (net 7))
 (segment (start 131.13641 101) (end 134 98.13641) (width 0.25) (layer F.Cu) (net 7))
 (segment (start 119.96 101) (end 131.13641 101) (width 0.25) (layer F.Cu) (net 7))
 (via (at 134 94) (size 0.8) (drill 0.4) (layers F.Cu B.Cu) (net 7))
 (segment (start 134 98.13641) (end 134 94) (width 0.25) (layer F.Cu) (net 7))
 (segment (start 134 94) (end 134 93) (width 0.25) (layer B.Cu) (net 7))
 (via (at 132.5 91.5) (size 0.8) (drill 0.4) (layers F.Cu B.Cu) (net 7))
 (segment (start 134 93) (end 132.5 91.5) (width 0.25) (layer B.Cu) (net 7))
 (segment (start 132.75 91.25) (end 132.75 90.75) (width 0.25) (layer F.Cu) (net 7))
 (segment (start 132.5 91.5) (end 132.75 91.25) (width 0.25) (layer F.Cu) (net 7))
 (segment (start 132.75 90.75) (end 131 92.5) (width 0.25) (layer F.Cu) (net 7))
 (segment (start 135.5 88) (end 132.75 90.75) (width 0.25) (layer F.Cu) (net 7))
 (segment (start 145.5 86) (end 145.5 88) (width 0.25) (layer F.Cu) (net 8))
 (segment (start 138.5 88) (end 138.5 86) (width 0.25) (layer F.Cu) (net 9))
 (segment (start 142 88) (end 142 85.5) (width 0.25) (layer F.Cu) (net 10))
 (segment (start 127.275001 95.775001) (end 129 97.5) (width 0.25) (layer F.Cu) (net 15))
 (segment (start 115.5 91.46) (end 123.04 99) (width 0.25) (layer F.Cu) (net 15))
 (segment (start 123.04 99) (end 128.5 99) (width 0.25) (layer F.Cu) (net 15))
 (segment (start 129 98.5) (end 129 97.5) (width 0.25) (layer F.Cu) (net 15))
 (segment (start 128.5 99) (end 129 98.5) (width 0.25) (layer F.Cu) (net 15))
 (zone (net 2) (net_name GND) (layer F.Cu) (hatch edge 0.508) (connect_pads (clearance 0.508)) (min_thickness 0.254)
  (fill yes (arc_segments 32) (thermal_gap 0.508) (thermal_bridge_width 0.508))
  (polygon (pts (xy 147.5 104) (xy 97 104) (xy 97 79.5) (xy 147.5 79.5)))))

